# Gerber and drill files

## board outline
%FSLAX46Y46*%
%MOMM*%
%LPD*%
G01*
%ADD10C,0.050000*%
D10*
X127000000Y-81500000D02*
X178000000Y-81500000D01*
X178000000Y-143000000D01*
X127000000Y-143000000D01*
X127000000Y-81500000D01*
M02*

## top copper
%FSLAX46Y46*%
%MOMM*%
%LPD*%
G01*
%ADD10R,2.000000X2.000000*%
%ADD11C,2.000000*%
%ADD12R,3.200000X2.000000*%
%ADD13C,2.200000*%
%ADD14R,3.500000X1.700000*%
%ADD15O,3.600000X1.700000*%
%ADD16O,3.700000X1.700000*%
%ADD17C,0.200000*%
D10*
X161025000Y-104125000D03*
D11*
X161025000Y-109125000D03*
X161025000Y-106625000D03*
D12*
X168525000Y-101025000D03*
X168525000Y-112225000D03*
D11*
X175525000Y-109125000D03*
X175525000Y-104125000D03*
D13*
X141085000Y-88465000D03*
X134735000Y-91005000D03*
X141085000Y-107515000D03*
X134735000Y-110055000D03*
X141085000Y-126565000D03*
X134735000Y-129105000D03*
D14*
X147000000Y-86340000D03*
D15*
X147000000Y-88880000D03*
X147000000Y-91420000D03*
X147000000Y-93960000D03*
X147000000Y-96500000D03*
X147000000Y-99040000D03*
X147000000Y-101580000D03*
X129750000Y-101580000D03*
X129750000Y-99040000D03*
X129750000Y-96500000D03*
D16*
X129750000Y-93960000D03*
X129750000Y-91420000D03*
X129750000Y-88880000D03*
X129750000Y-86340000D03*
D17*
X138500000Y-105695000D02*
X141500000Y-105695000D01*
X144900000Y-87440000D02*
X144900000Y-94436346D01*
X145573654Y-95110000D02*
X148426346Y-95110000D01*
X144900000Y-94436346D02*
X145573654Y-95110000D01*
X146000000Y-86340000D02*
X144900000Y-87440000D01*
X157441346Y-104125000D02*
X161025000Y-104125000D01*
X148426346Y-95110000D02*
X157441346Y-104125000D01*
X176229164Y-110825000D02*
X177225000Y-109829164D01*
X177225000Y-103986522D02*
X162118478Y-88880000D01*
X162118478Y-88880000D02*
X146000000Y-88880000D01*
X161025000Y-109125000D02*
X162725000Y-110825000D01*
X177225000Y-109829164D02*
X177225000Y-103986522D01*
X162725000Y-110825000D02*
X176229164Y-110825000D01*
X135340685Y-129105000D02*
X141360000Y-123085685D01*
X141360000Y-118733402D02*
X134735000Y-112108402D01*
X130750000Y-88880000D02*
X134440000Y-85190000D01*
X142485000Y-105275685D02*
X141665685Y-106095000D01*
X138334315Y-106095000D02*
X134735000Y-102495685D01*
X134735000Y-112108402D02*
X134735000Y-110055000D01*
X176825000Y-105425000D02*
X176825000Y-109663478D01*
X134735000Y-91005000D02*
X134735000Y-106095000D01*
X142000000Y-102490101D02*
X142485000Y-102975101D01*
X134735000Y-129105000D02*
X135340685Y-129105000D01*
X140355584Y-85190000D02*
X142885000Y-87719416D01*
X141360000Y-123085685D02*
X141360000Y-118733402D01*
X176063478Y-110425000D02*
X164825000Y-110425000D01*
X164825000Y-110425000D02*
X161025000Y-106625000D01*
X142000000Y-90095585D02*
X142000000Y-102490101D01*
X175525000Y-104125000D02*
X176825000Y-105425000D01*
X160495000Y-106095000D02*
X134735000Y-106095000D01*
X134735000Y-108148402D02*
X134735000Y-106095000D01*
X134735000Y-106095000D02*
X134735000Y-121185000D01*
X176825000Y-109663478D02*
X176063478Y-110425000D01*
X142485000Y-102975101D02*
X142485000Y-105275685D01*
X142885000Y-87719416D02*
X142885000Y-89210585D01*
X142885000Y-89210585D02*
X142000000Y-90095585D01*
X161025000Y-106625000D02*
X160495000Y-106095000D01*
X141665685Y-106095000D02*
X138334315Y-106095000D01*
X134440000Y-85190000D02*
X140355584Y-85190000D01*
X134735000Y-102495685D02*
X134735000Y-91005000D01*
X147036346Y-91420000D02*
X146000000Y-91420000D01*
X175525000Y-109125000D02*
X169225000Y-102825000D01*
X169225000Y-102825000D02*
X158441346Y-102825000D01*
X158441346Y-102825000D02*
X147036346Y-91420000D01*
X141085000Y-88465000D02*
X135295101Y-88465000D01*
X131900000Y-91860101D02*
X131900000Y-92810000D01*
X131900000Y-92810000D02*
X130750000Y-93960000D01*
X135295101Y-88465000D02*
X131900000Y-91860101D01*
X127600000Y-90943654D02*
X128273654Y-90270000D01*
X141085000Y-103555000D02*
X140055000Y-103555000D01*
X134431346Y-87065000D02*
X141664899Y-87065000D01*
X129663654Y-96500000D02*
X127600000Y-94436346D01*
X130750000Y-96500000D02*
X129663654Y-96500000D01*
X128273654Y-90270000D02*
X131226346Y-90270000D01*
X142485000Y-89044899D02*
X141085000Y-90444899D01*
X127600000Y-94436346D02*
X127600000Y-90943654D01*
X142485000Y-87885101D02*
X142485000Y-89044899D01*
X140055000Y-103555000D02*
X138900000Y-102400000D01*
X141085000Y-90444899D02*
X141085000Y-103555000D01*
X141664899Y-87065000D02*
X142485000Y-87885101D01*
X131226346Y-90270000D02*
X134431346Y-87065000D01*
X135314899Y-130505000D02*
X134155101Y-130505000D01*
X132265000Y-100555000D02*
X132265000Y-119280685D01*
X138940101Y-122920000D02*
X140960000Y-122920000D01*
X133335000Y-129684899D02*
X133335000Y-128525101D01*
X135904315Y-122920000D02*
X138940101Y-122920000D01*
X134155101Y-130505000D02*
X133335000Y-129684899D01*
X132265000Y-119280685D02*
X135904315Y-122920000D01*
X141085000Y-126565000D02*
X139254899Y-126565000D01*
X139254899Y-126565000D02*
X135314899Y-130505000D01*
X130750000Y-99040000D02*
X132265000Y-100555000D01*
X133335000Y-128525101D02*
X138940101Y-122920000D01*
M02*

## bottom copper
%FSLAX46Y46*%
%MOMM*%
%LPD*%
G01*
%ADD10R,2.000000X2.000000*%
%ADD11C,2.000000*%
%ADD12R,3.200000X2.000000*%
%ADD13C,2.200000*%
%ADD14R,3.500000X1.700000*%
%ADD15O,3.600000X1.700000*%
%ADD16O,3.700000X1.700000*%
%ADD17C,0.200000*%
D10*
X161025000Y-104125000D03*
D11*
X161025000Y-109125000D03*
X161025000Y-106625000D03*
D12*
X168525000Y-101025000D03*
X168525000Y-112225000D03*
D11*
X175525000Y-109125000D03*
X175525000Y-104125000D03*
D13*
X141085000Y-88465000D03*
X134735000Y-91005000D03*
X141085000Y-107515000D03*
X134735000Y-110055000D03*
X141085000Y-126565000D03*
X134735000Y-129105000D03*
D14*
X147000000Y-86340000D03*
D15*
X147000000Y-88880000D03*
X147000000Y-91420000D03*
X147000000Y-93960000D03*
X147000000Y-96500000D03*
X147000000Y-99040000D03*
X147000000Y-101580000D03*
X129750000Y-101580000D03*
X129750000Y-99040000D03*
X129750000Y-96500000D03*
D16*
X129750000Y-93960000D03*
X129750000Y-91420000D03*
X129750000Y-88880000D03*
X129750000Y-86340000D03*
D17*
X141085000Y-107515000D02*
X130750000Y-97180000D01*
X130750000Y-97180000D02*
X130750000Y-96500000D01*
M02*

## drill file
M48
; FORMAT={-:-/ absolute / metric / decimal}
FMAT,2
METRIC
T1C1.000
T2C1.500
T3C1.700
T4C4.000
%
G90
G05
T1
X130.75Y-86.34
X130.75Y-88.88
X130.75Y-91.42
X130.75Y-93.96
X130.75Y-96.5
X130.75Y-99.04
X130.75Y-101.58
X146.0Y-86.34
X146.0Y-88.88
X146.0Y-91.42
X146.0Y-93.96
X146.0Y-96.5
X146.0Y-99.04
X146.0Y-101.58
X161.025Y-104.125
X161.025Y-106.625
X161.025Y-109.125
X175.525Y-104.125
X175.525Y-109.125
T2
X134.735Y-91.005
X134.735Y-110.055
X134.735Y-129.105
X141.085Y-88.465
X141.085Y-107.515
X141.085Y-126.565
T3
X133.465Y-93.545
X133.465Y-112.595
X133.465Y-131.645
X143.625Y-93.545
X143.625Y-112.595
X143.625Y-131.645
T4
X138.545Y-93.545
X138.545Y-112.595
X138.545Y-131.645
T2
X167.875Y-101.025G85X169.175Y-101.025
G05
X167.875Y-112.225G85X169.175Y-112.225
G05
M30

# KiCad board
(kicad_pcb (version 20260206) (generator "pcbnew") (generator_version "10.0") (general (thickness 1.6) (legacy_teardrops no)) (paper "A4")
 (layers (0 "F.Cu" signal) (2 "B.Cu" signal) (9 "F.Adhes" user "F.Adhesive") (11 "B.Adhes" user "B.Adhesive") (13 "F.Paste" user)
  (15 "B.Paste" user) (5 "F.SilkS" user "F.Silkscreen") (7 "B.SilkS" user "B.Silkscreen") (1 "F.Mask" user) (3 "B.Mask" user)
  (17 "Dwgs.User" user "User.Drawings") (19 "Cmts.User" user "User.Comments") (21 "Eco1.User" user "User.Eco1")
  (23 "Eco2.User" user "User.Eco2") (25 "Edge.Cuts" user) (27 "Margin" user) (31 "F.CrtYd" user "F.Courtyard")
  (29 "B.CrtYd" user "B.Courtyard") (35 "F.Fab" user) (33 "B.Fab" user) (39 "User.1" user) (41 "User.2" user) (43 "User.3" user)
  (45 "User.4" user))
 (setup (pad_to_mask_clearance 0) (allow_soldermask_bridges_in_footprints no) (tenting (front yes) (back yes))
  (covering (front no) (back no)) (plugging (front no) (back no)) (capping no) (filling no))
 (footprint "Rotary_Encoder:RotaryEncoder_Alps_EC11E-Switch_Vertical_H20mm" (layer "F.Cu") (at 161.025 104.125)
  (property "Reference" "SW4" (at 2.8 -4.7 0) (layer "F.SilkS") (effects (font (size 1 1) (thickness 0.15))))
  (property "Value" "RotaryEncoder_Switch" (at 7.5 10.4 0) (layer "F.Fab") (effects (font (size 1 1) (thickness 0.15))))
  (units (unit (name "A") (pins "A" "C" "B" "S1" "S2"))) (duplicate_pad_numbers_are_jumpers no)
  (pad "A" thru_hole rect (at 0 0) (size 2 2) (drill 1) (layers "*.Cu" "*.Mask") (remove_unused_layers no) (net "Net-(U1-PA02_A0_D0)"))
  (pad "B" thru_hole circle (at 0 5) (size 2 2) (drill 1) (layers "*.Cu" "*.Mask") (remove_unused_layers no) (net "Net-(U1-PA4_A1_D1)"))
  (pad "C" thru_hole circle (at 0 2.5) (size 2 2) (drill 1) (layers "*.Cu" "*.Mask") (remove_unused_layers no) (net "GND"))
  (pad "MP" thru_hole rect (at 7.5 -3.1) (size 3.2 2) (drill oval 2.8 1.5) (layers "*.Cu" "*.Mask") (remove_unused_layers no))
  (pad "MP" thru_hole rect (at 7.5 8.1) (size 3.2 2) (drill oval 2.8 1.5) (layers "*.Cu" "*.Mask") (remove_unused_layers no))
  (pad "S1" thru_hole circle (at 14.5 5) (size 2 2) (drill 1) (layers "*.Cu" "*.Mask") (remove_unused_layers no) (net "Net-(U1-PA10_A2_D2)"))
  (pad "S2" thru_hole circle (at 14.5 0) (size 2 2) (drill 1) (layers "*.Cu" "*.Mask") (remove_unused_layers no) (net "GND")))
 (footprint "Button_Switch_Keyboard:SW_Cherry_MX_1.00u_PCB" (layer "F.Cu") (at 141.085 88.465)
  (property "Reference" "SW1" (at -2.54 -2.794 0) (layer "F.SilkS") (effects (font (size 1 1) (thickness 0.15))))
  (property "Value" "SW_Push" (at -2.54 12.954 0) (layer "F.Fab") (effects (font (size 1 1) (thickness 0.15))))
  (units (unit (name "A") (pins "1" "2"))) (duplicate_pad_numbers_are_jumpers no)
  (pad "" np_thru_hole circle (at -7.62 5.08) (size 1.7 1.7) (drill 1.7) (layers "*.Cu" "*.Mask"))
  (pad "" np_thru_hole circle (at -2.54 5.08) (size 4 4) (drill 4) (layers "*.Cu" "*.Mask"))
  (pad "" np_thru_hole circle (at 2.54 5.08) (size 1.7 1.7) (drill 1.7) (layers "*.Cu" "*.Mask"))
  (pad "1" thru_hole circle (at 0 0) (size 2.2 2.2) (drill 1.5) (layers "*.Cu" "*.Mask") (remove_unused_layers no)
   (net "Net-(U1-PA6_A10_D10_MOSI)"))
  (pad "2" thru_hole circle (at -6.35 2.54) (size 2.2 2.2) (drill 1.5) (layers "*.Cu" "*.Mask") (remove_unused_layers no) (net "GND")))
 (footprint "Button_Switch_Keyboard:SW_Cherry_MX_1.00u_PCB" (layer "F.Cu") (at 141.085 107.515)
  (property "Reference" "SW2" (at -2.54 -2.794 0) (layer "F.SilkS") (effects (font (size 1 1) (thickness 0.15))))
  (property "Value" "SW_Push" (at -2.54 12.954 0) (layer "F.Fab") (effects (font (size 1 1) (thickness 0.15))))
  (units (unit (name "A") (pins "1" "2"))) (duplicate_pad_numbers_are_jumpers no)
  (pad "" np_thru_hole circle (at -7.62 5.08) (size 1.7 1.7) (drill 1.7) (layers "*.Cu" "*.Mask"))
  (pad "" np_thru_hole circle (at -2.54 5.08) (size 4 4) (drill 4) (layers "*.Cu" "*.Mask"))
  (pad "" np_thru_hole circle (at 2.54 5.08) (size 1.7 1.7) (drill 1.7) (layers "*.Cu" "*.Mask"))
  (pad "1" thru_hole circle (at 0 0) (size 2.2 2.2) (drill 1.5) (layers "*.Cu" "*.Mask") (remove_unused_layers no)
   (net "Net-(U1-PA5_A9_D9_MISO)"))
  (pad "2" thru_hole circle (at -6.35 2.54) (size 2.2 2.2) (drill 1.5) (layers "*.Cu" "*.Mask") (remove_unused_layers no) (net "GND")))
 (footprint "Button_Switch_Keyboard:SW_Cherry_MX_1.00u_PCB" (layer "F.Cu") (at 141.085 126.565)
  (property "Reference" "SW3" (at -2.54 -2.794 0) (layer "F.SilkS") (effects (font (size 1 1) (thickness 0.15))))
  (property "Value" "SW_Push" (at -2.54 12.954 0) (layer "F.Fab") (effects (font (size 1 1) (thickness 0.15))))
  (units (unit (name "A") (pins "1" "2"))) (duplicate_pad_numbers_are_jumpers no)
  (pad "" np_thru_hole circle (at -7.62 5.08) (size 1.7 1.7) (drill 1.7) (layers "*.Cu" "*.Mask"))
  (pad "" np_thru_hole circle (at -2.54 5.08) (size 4 4) (drill 4) (layers "*.Cu" "*.Mask"))
  (pad "" np_thru_hole circle (at 2.54 5.08) (size 1.7 1.7) (drill 1.7) (layers "*.Cu" "*.Mask"))
  (pad "1" thru_hole circle (at 0 0) (size 2.2 2.2) (drill 1.5) (layers "*.Cu" "*.Mask") (remove_unused_layers no)
   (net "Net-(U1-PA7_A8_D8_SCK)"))
  (pad "2" thru_hole circle (at -6.35 2.54) (size 2.2 2.2) (drill 1.5) (layers "*.Cu" "*.Mask") (remove_unused_layers no) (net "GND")))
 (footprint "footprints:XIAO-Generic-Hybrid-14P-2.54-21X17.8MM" (layer "B.Cu") (at 138.375 93.96 180)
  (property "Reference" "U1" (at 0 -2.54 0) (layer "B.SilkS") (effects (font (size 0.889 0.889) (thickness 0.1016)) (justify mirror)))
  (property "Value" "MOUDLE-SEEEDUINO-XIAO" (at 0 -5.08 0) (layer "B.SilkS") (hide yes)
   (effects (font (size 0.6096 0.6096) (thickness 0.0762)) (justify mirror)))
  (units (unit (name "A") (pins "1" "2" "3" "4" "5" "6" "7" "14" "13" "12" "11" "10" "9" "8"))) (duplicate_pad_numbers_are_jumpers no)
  (pad "1" thru_hole rect (at -7.625 7.62 180) (size 3.5 1.7) (drill 1 (offset -1 0)) (layers "*.Cu" "*.Mask") (remove_unused_layers no)
   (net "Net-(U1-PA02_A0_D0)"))
  (pad "2" thru_hole oval (at -7.625 5.08 180) (size 3.6 1.7) (drill 1 (offset -1 0)) (layers "*.Cu" "*.Mask") (remove_unused_layers no)
   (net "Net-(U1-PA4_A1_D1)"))
  (pad "3" thru_hole oval (at -7.625 2.54 180) (size 3.6 1.7) (drill 1 (offset -1 0)) (layers "*.Cu" "*.Mask") (remove_unused_layers no)
   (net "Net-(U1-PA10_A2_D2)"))
  (pad "4" thru_hole oval (at -7.625 0 180) (size 3.6 1.7) (drill 1 (offset -1 0)) (layers "*.Cu" "*.Mask") (remove_unused_layers no)
   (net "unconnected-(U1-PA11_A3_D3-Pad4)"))
  (pad "5" thru_hole oval (at -7.625 -2.54 180) (size 3.6 1.7) (drill 1 (offset -1 0)) (layers "*.Cu" "*.Mask") (remove_unused_layers no)
   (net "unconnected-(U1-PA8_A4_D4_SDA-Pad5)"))
  (pad "6" thru_hole oval (at -7.625 -5.08) (size 3.6 1.7) (drill 1 (offset 1 0)) (layers "*.Cu" "*.Mask") (remove_unused_layers no)
   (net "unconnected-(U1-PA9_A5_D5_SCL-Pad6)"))
  (pad "7" thru_hole oval (at -7.625 -7.62 180) (size 3.6 1.7) (drill 1 (offset -1 0)) (layers "*.Cu" "*.Mask") (remove_unused_layers no)
   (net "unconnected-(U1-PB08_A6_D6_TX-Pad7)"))
  (pad "8" thru_hole oval (at 7.625 -7.62 180) (size 3.6 1.7) (drill 1 (offset 1 0)) (layers "*.Cu" "*.Mask") (remove_unused_layers no)
   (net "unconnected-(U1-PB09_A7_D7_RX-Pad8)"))
  (pad "9" thru_hole oval (at 7.625 -5.08 180) (size 3.6 1.7) (drill 1 (offset 1 0)) (layers "*.Cu" "*.Mask") (remove_unused_layers no)
   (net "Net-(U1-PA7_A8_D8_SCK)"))
  (pad "10" thru_hole oval (at 7.625 -2.54 180) (size 3.6 1.7) (drill 1 (offset 1 0)) (layers "*.Cu" "*.Mask") (remove_unused_layers no)
   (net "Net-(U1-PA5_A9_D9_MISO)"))
  (pad "11" thru_hole oval (at 7.625 0 180) (size 3.7 1.7) (drill 1 (offset 1 0)) (layers "*.Cu" "*.Mask") (remove_unused_layers no)
   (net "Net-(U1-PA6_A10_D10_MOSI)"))
  (pad "12" thru_hole oval (at 7.625 2.54 180) (size 3.7 1.7) (drill 1 (offset 1 0)) (layers "*.Cu" "*.Mask") (remove_unused_layers no)
   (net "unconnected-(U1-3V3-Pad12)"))
  (pad "13" thru_hole oval (at 7.625 5.08 180) (size 3.7 1.7) (drill 1 (offset 1 0)) (layers "*.Cu" "*.Mask") (remove_unused_layers no)
   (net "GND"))
  (pad "14" thru_hole oval (at 7.625 7.62 180) (size 3.7 1.7) (drill 1 (offset 1 0)) (layers "*.Cu" "*.Mask") (remove_unused_layers no)
   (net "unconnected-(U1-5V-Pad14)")))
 (gr_rect (start 127 81.5) (end 178 143) (stroke (width 0.05) (type solid)) (fill no) (layer "Edge.Cuts"))
 (segment (start 138.5 105.695) (end 141.5 105.695) (width 0.2) (layer "F.Cu") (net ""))
 (segment (start 144.9 87.44) (end 144.9 94.436346) (width 0.2) (layer "F.Cu") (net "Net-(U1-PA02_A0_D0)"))
 (segment (start 145.573654 95.11) (end 148.426346 95.11) (width 0.2) (layer "F.Cu") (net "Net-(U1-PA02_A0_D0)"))
 (segment (start 144.9 94.436346) (end 145.573654 95.11) (width 0.2) (layer "F.Cu") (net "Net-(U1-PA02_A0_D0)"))
 (segment (start 146 86.34) (end 144.9 87.44) (width 0.2) (layer "F.Cu") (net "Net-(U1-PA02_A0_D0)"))
 (segment (start 157.441346 104.125) (end 161.025 104.125) (width 0.2) (layer "F.Cu") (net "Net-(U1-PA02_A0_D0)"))
 (segment (start 148.426346 95.11) (end 157.441346 104.125) (width 0.2) (layer "F.Cu") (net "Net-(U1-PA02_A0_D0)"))
 (segment (start 176.229164 110.825) (end 177.225 109.829164) (width 0.2) (layer "F.Cu") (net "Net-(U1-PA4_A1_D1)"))
 (segment (start 177.225 103.986522) (end 162.118478 88.88) (width 0.2) (layer "F.Cu") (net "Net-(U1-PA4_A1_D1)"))
 (segment (start 162.118478 88.88) (end 146 88.88) (width 0.2) (layer "F.Cu") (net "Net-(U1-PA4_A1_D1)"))
 (segment (start 161.025 109.125) (end 162.725 110.825) (width 0.2) (layer "F.Cu") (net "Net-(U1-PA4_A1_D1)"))
 (segment (start 177.225 109.829164) (end 177.225 103.986522) (width 0.2) (layer "F.Cu") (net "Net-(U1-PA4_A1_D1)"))
 (segment (start 162.725 110.825) (end 176.229164 110.825) (width 0.2) (layer "F.Cu") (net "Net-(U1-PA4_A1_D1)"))
 (segment (start 135.340685 129.105) (end 141.36 123.085685) (width 0.2) (layer "F.Cu") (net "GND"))
 (segment (start 141.36 118.733402) (end 134.735 112.108402) (width 0.2) (layer "F.Cu") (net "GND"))
 (segment (start 130.75 88.88) (end 134.44 85.19) (width 0.2) (layer "F.Cu") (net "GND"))
 (segment (start 142.485 105.275685) (end 141.665685 106.095) (width 0.2) (layer "F.Cu") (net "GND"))
 (segment (start 138.334315 106.095) (end 134.735 102.495685) (width 0.2) (layer "F.Cu") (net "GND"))
 (segment (start 134.735 112.108402) (end 134.735 110.055) (width 0.2) (layer "F.Cu") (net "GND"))
 (segment (start 176.825 105.425) (end 176.825 109.663478) (width 0.2) (layer "F.Cu") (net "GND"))
 (segment (start 134.735 91.005) (end 134.735 106.095) (width 0.2) (layer "F.Cu") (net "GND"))
 (segment (start 142 102.490101) (end 142.485 102.975101) (width 0.2) (layer "F.Cu") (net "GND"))
 (segment (start 134.735 129.105) (end 135.340685 129.105) (width 0.2) (layer "F.Cu") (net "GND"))
 (segment (start 140.355584 85.19) (end 142.885 87.719416) (width 0.2) (layer "F.Cu") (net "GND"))
 (segment (start 141.36 123.085685) (end 141.36 118.733402) (width 0.2) (layer "F.Cu") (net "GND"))
 (segment (start 176.063478 110.425) (end 164.825 110.425) (width 0.2) (layer "F.Cu") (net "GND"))
 (segment (start 164.825 110.425) (end 161.025 106.625) (width 0.2) (layer "F.Cu") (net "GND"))
 (segment (start 142 90.095585) (end 142 102.490101) (width 0.2) (layer "F.Cu") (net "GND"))
 (segment (start 175.525 104.125) (end 176.825 105.425) (width 0.2) (layer "F.Cu") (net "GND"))
 (segment (start 160.495 106.095) (end 134.735 106.095) (width 0.2) (layer "F.Cu") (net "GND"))
 (segment (start 134.735 108.148402) (end 134.735 106.095) (width 0.2) (layer "F.Cu") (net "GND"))
 (segment (start 134.735 106.095) (end 134.735 121.185) (width 0.2) (layer "F.Cu") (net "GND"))
 (segment (start 176.825 109.663478) (end 176.063478 110.425) (width 0.2) (layer "F.Cu") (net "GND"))
 (segment (start 142.485 102.975101) (end 142.485 105.275685) (width 0.2) (layer "F.Cu") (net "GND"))
 (segment (start 142.885 87.719416) (end 142.885 89.210585) (width 0.2) (layer "F.Cu") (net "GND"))
 (segment (start 142.885 89.210585) (end 142 90.095585) (width 0.2) (layer "F.Cu") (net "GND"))
 (segment (start 161.025 106.625) (end 160.495 106.095) (width 0.2) (layer "F.Cu") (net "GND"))
 (segment (start 141.665685 106.095) (end 138.334315 106.095) (width 0.2) (layer "F.Cu") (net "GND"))
 (segment (start 134.44 85.19) (end 140.355584 85.19) (width 0.2) (layer "F.Cu") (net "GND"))
 (segment (start 134.735 102.495685) (end 134.735 91.005) (width 0.2) (layer "F.Cu") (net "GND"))
 (segment (start 147.036346 91.42) (end 146 91.42) (width 0.2) (layer "F.Cu") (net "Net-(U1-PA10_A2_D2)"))
 (segment (start 175.525 109.125) (end 169.225 102.825) (width 0.2) (layer "F.Cu") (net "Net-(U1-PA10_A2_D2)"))
 (segment (start 169.225 102.825) (end 158.441346 102.825) (width 0.2) (layer "F.Cu") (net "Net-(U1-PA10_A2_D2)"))
 (segment (start 158.441346 102.825) (end 147.036346 91.42) (width 0.2) (layer "F.Cu") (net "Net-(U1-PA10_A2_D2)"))
 (segment (start 141.085 88.465) (end 135.295101 88.465) (width 0.2) (layer "F.Cu") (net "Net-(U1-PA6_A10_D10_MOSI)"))
 (segment (start 131.9 91.860101) (end 131.9 92.81) (width 0.2) (layer "F.Cu") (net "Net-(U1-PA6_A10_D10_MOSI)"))
 (segment (start 131.9 92.81) (end 130.75 93.96) (width 0.2) (layer "F.Cu") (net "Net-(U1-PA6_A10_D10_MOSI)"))
 (segment (start 135.295101 88.465) (end 131.9 91.860101) (width 0.2) (layer "F.Cu") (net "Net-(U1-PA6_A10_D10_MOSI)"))
 (segment (start 127.6 90.943654) (end 128.273654 90.27) (width 0.2) (layer "F.Cu") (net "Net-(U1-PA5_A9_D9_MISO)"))
 (segment (start 141.085 103.555) (end 140.055 103.555) (width 0.2) (layer "F.Cu") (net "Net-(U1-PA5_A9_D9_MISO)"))
 (segment (start 134.431346 87.065) (end 141.664899 87.065) (width 0.2) (layer "F.Cu") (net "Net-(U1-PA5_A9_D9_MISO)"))
 (segment (start 129.663654 96.5) (end 127.6 94.436346) (width 0.2) (layer "F.Cu") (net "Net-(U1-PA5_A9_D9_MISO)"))
 (segment (start 130.75 96.5) (end 129.663654 96.5) (width 0.2) (layer "F.Cu") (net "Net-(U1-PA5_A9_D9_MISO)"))
 (segment (start 128.273654 90.27) (end 131.226346 90.27) (width 0.2) (layer "F.Cu") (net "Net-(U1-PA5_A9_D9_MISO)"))
 (segment (start 142.485 89.044899) (end 141.085 90.444899) (width 0.2) (layer "F.Cu") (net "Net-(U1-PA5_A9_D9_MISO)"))
 (segment (start 127.6 94.436346) (end 127.6 90.943654) (width 0.2) (layer "F.Cu") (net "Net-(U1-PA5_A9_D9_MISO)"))
 (segment (start 142.485 87.885101) (end 142.485 89.044899) (width 0.2) (layer "F.Cu") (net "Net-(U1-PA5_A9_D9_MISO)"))
 (segment (start 140.055 103.555) (end 138.9 102.4) (width 0.2) (layer "F.Cu") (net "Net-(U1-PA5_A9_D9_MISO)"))
 (segment (start 141.085 90.444899) (end 141.085 103.555) (width 0.2) (layer "F.Cu") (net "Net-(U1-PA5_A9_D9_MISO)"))
 (segment (start 141.664899 87.065) (end 142.485 87.885101) (width 0.2) (layer "F.Cu") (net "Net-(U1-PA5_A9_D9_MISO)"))
 (segment (start 131.226346 90.27) (end 134.431346 87.065) (width 0.2) (layer "F.Cu") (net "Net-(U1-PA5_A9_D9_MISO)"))
 (segment (start 141.085 107.515) (end 130.75 97.18) (width 0.2) (layer "B.Cu") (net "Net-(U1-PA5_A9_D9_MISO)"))
 (segment (start 130.75 97.18) (end 130.75 96.5) (width 0.2) (layer "B.Cu") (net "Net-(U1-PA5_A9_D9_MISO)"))
 (segment (start 135.314899 130.505) (end 134.155101 130.505) (width 0.2) (layer "F.Cu") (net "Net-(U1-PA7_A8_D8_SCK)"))
 (segment (start 132.265 100.555) (end 132.265 119.280685) (width 0.2) (layer "F.Cu") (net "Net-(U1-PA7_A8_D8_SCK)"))
 (segment (start 138.940101 122.92) (end 140.96 122.92) (width 0.2) (layer "F.Cu") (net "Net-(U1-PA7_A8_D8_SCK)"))
 (segment (start 133.335 129.684899) (end 133.335 128.525101) (width 0.2) (layer "F.Cu") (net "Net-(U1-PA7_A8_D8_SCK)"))
 (segment (start 135.904315 122.92) (end 138.940101 122.92) (width 0.2) (layer "F.Cu") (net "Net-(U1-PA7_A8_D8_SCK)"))
 (segment (start 134.155101 130.505) (end 133.335 129.684899) (width 0.2) (layer "F.Cu") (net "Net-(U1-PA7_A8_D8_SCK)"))
 (segment (start 132.265 119.280685) (end 135.904315 122.92) (width 0.2) (layer "F.Cu") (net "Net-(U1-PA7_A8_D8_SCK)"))
 (segment (start 141.085 126.565) (end 139.254899 126.565) (width 0.2) (layer "F.Cu") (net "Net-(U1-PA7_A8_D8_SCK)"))
 (segment (start 139.254899 126.565) (end 135.314899 130.505) (width 0.2) (layer "F.Cu") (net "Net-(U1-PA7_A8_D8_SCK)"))
 (segment (start 130.75 99.04) (end 132.265 100.555) (width 0.2) (layer "F.Cu") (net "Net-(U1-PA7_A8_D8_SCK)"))
 (segment (start 133.335 128.525101) (end 138.940101 122.92) (width 0.2) (layer "F.Cu") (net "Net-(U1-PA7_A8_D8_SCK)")))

